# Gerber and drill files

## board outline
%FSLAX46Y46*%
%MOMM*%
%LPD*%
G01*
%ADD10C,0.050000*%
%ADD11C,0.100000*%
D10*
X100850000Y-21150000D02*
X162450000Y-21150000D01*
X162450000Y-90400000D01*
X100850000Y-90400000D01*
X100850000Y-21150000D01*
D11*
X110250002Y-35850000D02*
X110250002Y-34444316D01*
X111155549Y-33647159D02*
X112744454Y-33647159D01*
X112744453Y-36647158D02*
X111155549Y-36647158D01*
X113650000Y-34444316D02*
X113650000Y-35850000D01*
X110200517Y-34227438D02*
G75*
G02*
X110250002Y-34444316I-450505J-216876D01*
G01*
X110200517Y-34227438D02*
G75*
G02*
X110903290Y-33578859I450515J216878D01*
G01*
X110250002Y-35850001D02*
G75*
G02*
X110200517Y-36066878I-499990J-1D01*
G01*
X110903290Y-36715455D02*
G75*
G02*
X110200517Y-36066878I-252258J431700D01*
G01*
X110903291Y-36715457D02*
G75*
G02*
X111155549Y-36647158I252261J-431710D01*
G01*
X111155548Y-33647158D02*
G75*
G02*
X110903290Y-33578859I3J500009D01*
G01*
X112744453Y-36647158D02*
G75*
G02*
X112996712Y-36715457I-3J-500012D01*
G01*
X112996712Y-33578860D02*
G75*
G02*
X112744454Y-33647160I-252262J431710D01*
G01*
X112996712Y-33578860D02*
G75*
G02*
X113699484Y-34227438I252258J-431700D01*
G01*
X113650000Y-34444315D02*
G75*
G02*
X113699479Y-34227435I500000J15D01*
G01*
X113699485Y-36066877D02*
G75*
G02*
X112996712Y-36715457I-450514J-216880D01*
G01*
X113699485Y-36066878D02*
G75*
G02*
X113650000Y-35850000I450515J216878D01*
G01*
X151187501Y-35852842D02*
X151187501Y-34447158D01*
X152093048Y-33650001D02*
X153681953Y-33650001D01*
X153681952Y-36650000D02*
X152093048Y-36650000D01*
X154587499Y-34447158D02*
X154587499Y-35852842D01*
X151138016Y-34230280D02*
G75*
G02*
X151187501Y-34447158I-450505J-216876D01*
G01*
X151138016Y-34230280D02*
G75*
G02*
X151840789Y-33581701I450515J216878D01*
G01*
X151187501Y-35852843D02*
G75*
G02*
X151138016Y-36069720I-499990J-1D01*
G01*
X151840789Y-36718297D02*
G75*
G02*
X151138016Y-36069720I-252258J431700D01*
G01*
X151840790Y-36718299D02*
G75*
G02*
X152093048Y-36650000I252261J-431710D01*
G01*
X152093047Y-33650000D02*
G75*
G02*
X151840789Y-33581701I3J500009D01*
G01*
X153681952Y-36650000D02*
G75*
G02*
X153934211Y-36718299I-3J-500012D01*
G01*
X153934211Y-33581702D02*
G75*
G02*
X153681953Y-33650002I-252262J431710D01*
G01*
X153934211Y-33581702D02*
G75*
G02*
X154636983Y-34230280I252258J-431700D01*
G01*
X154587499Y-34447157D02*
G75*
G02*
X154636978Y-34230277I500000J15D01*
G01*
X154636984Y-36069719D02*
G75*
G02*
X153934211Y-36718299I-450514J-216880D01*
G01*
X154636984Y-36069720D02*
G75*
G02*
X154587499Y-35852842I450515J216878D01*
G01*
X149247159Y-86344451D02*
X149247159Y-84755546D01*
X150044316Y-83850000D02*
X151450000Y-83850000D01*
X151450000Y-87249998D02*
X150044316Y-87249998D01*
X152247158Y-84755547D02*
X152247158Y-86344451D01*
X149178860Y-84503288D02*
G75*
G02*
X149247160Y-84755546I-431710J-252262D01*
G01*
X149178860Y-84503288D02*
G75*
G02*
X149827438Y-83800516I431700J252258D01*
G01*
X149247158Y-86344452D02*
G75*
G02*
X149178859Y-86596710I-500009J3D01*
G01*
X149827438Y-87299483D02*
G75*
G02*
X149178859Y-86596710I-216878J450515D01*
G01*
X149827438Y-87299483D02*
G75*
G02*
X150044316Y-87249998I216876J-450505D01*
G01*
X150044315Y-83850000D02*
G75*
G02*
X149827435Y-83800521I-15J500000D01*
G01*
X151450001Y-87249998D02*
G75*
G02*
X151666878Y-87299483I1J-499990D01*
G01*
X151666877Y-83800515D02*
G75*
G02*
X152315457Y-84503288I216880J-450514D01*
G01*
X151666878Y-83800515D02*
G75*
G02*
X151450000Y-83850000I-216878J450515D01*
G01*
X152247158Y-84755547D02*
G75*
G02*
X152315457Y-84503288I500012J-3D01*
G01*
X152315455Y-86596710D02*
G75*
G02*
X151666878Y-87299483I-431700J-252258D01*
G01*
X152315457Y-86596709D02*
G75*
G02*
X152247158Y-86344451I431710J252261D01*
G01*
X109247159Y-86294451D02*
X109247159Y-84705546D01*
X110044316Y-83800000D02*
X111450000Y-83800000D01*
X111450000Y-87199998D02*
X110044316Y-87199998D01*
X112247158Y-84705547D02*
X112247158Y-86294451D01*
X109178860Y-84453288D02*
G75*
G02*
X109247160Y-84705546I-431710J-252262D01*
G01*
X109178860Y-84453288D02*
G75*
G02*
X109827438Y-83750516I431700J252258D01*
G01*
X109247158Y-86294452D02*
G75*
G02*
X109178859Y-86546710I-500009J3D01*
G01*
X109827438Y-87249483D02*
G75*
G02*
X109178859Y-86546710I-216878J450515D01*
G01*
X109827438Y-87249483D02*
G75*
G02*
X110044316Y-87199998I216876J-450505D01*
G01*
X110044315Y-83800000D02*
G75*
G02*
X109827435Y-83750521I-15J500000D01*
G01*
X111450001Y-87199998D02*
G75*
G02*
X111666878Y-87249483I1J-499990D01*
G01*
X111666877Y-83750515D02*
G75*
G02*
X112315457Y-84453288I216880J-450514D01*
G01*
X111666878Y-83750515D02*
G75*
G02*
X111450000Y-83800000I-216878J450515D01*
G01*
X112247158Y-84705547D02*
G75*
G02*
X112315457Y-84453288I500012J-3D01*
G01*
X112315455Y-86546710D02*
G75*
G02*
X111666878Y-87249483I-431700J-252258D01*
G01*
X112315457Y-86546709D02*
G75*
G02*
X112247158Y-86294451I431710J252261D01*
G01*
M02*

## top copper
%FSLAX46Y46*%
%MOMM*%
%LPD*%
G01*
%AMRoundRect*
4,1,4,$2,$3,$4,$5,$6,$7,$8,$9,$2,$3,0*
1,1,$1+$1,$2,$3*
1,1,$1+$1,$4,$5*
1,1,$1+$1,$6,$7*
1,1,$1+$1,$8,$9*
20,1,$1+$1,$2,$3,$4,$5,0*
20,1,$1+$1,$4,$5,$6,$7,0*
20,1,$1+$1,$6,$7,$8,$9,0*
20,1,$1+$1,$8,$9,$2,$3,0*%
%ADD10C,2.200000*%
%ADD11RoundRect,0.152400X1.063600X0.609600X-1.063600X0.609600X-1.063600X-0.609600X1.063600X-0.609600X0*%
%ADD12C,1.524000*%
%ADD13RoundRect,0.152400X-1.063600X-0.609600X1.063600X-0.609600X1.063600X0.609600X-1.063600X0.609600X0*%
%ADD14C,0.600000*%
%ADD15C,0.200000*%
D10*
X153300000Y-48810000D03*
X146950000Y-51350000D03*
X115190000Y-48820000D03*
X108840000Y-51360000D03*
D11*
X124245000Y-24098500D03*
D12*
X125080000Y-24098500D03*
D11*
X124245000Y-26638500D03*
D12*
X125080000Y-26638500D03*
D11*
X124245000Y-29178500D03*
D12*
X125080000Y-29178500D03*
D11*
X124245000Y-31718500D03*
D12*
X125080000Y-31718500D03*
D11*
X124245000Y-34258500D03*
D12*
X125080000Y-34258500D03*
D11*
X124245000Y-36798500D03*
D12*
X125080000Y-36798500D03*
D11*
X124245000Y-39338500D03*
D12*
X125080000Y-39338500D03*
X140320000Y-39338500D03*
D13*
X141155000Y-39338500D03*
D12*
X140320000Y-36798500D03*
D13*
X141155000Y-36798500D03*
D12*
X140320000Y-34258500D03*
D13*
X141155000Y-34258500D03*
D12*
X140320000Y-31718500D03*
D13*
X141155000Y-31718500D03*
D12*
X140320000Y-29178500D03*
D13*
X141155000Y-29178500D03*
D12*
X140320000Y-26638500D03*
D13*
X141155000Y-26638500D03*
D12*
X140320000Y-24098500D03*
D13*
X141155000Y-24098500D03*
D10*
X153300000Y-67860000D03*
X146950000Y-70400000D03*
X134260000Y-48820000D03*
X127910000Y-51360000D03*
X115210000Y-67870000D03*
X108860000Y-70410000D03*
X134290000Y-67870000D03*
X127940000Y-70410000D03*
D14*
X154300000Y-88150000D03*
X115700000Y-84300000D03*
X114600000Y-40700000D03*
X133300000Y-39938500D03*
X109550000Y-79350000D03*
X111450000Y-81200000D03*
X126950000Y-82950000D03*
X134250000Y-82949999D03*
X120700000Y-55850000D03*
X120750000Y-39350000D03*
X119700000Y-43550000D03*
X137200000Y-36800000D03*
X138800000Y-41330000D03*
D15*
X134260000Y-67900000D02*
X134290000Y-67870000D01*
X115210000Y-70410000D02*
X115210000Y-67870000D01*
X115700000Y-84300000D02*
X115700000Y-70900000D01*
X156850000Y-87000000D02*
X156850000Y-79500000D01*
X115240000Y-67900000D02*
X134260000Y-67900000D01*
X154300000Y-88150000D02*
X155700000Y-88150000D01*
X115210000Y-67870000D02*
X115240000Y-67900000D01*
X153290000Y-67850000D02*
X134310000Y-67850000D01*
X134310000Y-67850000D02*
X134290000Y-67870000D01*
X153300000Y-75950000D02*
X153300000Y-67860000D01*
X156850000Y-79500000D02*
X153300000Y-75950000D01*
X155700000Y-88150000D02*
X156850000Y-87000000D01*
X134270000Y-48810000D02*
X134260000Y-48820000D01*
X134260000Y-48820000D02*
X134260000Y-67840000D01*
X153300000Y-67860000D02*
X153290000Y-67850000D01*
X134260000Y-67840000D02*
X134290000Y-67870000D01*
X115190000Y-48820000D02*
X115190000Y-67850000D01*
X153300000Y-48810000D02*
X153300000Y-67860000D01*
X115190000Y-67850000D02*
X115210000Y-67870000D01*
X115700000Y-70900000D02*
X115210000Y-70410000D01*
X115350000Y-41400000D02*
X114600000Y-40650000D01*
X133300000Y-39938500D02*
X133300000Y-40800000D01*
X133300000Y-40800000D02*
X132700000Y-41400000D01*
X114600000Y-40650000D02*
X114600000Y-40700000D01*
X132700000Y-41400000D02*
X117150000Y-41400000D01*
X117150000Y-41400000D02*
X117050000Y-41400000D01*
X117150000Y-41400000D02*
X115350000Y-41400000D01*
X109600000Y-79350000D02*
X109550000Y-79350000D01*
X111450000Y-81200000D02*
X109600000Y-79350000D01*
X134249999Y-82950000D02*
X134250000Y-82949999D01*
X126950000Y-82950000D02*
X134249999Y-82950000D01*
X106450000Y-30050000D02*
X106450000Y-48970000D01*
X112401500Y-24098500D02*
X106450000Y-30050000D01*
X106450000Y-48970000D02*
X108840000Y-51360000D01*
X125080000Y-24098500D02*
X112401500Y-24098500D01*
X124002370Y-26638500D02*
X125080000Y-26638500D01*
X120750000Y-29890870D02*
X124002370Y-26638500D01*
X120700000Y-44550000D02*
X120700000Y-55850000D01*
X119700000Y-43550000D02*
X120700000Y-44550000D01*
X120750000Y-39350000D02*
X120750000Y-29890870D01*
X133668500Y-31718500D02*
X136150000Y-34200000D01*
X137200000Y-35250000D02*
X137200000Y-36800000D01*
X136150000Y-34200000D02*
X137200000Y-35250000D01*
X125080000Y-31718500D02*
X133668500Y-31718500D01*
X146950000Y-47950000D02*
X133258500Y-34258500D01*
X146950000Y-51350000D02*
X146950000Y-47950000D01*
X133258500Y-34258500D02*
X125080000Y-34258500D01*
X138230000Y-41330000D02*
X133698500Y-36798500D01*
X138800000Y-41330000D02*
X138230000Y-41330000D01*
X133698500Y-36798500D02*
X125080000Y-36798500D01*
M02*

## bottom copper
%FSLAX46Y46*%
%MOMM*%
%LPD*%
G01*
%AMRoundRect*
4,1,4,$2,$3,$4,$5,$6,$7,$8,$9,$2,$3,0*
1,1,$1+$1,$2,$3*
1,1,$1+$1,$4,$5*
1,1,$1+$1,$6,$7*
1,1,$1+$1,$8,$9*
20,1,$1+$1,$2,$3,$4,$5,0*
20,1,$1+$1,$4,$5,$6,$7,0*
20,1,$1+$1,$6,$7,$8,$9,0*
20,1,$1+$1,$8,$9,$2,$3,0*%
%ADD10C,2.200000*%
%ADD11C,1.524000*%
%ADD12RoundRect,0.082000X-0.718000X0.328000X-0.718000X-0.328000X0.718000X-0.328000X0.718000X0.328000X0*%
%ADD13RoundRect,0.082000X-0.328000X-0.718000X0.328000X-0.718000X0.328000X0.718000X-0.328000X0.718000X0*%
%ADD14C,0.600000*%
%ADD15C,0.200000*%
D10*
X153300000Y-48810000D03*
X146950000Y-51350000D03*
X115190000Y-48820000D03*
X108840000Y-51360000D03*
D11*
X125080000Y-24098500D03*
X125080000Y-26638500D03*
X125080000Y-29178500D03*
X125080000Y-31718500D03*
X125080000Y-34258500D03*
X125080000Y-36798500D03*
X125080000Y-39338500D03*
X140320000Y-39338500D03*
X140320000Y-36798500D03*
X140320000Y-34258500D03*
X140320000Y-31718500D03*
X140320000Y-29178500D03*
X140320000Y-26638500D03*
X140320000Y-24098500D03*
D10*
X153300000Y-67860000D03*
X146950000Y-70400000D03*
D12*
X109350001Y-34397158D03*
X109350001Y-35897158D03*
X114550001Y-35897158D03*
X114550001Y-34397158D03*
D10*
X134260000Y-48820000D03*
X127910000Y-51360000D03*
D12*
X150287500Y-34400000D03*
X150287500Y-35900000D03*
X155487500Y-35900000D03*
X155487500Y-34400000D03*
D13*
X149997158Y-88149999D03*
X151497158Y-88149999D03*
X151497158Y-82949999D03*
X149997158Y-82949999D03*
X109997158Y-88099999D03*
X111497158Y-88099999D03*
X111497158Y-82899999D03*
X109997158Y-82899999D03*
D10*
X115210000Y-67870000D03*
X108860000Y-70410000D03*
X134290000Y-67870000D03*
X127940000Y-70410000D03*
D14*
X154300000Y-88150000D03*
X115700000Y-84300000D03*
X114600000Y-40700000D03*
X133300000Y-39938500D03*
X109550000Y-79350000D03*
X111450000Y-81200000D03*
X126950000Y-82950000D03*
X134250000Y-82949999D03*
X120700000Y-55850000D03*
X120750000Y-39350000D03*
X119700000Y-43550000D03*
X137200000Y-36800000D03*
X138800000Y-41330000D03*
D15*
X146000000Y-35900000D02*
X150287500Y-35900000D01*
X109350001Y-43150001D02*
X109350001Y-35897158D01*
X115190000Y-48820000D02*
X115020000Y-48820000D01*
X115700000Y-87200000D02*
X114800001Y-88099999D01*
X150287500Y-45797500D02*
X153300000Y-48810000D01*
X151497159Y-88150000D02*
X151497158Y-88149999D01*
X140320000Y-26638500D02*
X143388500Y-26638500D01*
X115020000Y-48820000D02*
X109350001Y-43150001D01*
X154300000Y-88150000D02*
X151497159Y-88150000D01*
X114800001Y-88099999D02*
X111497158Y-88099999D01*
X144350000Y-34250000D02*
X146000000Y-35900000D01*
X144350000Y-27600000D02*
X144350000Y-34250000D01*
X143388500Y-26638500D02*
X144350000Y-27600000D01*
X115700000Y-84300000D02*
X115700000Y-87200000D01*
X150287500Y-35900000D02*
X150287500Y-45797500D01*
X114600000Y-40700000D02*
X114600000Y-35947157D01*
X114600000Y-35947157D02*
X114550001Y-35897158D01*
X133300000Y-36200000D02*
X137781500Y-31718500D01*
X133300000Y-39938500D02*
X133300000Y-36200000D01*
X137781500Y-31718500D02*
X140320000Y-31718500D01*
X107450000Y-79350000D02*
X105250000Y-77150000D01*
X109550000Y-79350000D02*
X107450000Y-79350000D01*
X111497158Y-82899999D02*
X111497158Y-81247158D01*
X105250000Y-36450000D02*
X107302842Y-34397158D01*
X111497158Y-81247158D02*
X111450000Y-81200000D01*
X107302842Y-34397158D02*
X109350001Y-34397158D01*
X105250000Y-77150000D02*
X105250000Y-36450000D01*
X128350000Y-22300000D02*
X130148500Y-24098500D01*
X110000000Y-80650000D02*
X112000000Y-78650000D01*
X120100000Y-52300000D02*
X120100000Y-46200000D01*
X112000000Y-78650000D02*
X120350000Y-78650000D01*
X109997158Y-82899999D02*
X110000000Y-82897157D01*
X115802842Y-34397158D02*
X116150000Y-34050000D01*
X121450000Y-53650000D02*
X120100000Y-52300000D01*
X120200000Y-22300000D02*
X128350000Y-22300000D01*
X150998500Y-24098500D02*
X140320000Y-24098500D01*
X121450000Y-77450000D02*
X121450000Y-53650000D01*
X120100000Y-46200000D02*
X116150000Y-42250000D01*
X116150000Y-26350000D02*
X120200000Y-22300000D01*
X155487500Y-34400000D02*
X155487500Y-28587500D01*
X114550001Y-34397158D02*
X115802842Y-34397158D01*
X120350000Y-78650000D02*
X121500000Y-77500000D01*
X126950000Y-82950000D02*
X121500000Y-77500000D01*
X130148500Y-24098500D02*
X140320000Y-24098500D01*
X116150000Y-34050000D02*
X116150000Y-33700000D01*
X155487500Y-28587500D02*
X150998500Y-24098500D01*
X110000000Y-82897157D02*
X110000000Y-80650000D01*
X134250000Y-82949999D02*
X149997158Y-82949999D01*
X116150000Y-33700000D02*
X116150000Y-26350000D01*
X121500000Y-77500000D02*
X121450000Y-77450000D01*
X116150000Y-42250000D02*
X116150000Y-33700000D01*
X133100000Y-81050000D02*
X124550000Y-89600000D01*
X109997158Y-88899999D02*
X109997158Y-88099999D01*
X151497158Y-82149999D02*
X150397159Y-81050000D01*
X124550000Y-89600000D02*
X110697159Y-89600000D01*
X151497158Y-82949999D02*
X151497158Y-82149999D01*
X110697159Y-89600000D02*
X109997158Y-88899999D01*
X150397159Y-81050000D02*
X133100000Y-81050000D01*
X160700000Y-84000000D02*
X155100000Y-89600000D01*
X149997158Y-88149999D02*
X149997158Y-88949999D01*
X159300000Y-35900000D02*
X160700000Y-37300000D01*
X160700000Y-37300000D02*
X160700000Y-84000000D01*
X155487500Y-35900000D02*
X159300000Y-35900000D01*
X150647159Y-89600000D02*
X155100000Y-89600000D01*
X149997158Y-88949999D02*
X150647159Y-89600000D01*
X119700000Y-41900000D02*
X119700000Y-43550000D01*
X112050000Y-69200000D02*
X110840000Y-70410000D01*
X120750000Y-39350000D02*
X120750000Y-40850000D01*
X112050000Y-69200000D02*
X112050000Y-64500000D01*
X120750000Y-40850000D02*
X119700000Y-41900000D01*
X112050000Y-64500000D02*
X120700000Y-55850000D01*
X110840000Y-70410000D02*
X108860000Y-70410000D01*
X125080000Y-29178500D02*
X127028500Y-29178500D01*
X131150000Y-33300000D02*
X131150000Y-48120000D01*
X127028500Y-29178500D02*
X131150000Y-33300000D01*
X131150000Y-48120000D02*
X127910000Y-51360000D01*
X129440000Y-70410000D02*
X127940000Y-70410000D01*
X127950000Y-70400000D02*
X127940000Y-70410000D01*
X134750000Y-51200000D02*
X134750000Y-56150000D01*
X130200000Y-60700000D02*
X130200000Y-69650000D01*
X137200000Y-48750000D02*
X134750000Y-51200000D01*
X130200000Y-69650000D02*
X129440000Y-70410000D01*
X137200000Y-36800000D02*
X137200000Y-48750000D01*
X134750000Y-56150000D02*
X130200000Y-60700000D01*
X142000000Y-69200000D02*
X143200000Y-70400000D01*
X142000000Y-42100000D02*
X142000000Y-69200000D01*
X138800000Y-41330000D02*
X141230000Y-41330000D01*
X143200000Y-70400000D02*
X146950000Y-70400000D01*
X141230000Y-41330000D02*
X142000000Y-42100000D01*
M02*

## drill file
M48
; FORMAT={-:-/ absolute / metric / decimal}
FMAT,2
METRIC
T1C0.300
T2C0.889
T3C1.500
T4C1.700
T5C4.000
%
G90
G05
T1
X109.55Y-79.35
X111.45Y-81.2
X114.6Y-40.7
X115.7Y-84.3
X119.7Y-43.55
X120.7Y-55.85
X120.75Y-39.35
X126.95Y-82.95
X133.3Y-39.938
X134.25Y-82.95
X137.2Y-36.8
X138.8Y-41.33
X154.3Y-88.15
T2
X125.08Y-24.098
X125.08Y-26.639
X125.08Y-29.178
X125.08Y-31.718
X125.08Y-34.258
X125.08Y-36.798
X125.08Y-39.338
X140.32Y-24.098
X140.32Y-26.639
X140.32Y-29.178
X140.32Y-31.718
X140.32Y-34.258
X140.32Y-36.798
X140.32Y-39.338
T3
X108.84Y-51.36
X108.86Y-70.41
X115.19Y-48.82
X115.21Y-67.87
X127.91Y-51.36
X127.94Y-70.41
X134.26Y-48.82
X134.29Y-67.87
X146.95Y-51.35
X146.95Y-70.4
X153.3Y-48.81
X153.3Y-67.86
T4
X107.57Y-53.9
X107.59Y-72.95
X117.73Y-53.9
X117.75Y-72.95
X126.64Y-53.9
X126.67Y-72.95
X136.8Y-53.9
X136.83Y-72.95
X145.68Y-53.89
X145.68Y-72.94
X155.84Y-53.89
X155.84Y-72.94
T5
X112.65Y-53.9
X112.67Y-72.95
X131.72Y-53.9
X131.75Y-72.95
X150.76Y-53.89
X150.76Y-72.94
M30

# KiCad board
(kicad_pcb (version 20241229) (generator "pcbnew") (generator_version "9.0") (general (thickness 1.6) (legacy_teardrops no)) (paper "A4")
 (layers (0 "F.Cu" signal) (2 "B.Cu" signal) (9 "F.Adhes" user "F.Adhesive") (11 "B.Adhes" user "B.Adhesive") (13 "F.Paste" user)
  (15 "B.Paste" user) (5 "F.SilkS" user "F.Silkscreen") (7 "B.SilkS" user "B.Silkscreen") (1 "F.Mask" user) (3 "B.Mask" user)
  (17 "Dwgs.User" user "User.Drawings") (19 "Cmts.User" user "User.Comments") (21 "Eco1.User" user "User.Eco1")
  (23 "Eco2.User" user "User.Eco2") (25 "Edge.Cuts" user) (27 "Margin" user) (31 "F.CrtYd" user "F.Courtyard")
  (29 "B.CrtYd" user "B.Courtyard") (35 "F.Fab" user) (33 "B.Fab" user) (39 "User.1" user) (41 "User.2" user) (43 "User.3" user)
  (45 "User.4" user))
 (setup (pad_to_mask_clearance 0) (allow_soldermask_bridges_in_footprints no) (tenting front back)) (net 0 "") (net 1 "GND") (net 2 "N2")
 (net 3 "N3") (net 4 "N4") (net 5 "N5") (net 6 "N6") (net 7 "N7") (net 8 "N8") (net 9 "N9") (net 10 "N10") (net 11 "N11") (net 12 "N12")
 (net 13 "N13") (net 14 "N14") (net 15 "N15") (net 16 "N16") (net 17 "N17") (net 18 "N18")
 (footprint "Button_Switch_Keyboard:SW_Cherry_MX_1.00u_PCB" (layer "F.Cu") (at 153.3 48.81)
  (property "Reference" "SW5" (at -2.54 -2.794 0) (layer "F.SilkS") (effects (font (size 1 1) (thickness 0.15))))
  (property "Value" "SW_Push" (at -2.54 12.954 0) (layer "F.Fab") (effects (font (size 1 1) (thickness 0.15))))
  (pad "" np_thru_hole circle (at -7.62 5.08) (size 1.7 1.7) (drill 1.7) (layers "*.Cu" "*.Mask"))
  (pad "" np_thru_hole circle (at -2.54 5.08) (size 4 4) (drill 4) (layers "*.Cu" "*.Mask"))
  (pad "" np_thru_hole circle (at 2.54 5.08) (size 1.7 1.7) (drill 1.7) (layers "*.Cu" "*.Mask"))
  (pad "1" thru_hole circle (at 0 0) (size 2.2 2.2) (drill 1.5) (layers "*.Cu" "*.Mask") (remove_unused_layers no) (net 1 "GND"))
  (pad "2" thru_hole circle (at -6.35 2.54) (size 2.2 2.2) (drill 1.5) (layers "*.Cu" "*.Mask") (remove_unused_layers no) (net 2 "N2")))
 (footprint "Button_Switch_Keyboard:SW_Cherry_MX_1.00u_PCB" (layer "F.Cu") (at 115.19 48.82)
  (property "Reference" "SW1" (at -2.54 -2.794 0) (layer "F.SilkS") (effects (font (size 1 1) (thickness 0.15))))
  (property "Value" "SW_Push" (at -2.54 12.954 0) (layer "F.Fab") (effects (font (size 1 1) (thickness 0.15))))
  (pad "" np_thru_hole circle (at -7.62 5.08) (size 1.7 1.7) (drill 1.7) (layers "*.Cu" "*.Mask"))
  (pad "" np_thru_hole circle (at -2.54 5.08) (size 4 4) (drill 4) (layers "*.Cu" "*.Mask"))
  (pad "" np_thru_hole circle (at 2.54 5.08) (size 1.7 1.7) (drill 1.7) (layers "*.Cu" "*.Mask"))
  (pad "1" thru_hole circle (at 0 0) (size 2.2 2.2) (drill 1.5) (layers "*.Cu" "*.Mask") (remove_unused_layers no) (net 1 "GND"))
  (pad "2" thru_hole circle (at -6.35 2.54) (size 2.2 2.2) (drill 1.5) (layers "*.Cu" "*.Mask") (remove_unused_layers no) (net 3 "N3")))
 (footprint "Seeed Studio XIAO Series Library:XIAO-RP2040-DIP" (layer "F.Cu") (at 132.7 31.7185)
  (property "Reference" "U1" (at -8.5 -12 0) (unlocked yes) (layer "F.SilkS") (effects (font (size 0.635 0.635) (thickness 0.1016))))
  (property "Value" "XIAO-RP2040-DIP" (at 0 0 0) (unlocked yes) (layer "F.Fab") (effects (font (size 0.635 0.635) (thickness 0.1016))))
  (pad "1" smd roundrect (at -8.455 -7.62 180) (size 2.432 1.524) (layers "F.Cu" "F.Mask") (roundrect_rratio 0.1) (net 3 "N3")
   (thermal_bridge_angle 45))
  (pad "1" thru_hole circle (at -7.62 -7.62 180) (size 1.524 1.524) (drill 0.889) (layers "*.Cu" "*.Mask") (remove_unused_layers no)
   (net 3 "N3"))
  (pad "2" smd roundrect (at -8.455 -5.08 180) (size 2.432 1.524) (layers "F.Cu" "F.Mask") (roundrect_rratio 0.1) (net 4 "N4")
   (thermal_bridge_angle 45))
  (pad "2" thru_hole circle (at -7.62 -5.08 180) (size 1.524 1.524) (drill 0.889) (layers "*.Cu" "*.Mask") (remove_unused_layers no)
   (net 4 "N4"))
  (pad "3" smd roundrect (at -8.455 -2.54 180) (size 2.432 1.524) (layers "F.Cu" "F.Mask") (roundrect_rratio 0.1) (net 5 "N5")
   (thermal_bridge_angle 45))
  (pad "3" thru_hole circle (at -7.62 -2.54 180) (size 1.524 1.524) (drill 0.889) (layers "*.Cu" "*.Mask") (remove_unused_layers no)
   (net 5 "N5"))
  (pad "4" smd roundrect (at -8.455 0 180) (size 2.432 1.524) (layers "F.Cu" "F.Mask") (roundrect_rratio 0.1) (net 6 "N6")
   (thermal_bridge_angle 45))
  (pad "4" thru_hole circle (at -7.62 0 180) (size 1.524 1.524) (drill 0.889) (layers "*.Cu" "*.Mask") (remove_unused_layers no)
   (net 6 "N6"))
  (pad "5" smd roundrect (at -8.455 2.54 180) (size 2.432 1.524) (layers "F.Cu" "F.Mask") (roundrect_rratio 0.1) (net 2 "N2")
   (thermal_bridge_angle 45))
  (pad "5" thru_hole circle (at -7.62 2.54 180) (size 1.524 1.524) (drill 0.889) (layers "*.Cu" "*.Mask") (remove_unused_layers no)
   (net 2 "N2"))
  (pad "6" smd roundrect (at -8.455 5.08 180) (size 2.432 1.524) (layers "F.Cu" "F.Mask") (roundrect_rratio 0.1) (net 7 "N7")
   (thermal_bridge_angle 45))
  (pad "6" thru_hole circle (at -7.62 5.08 180) (size 1.524 1.524) (drill 0.889) (layers "*.Cu" "*.Mask") (remove_unused_layers no)
   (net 7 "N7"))
  (pad "7" smd roundrect (at -8.455 7.62 180) (size 2.432 1.524) (layers "F.Cu" "F.Mask") (roundrect_rratio 0.1) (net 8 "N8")
   (thermal_bridge_angle 45))
  (pad "7" thru_hole circle (at -7.62 7.62 180) (size 1.524 1.524) (drill 0.889) (layers "*.Cu" "*.Mask") (remove_unused_layers no)
   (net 8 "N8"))
  (pad "8" thru_hole circle (at 7.62 7.62) (size 1.524 1.524) (drill 0.889) (layers "*.Cu" "*.Mask") (remove_unused_layers no) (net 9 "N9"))
  (pad "8" smd roundrect (at 8.455 7.62) (size 2.432 1.524) (layers "F.Cu" "F.Mask") (roundrect_rratio 0.1) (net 9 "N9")
   (thermal_bridge_angle 45))
  (pad "9" thru_hole circle (at 7.62 5.08) (size 1.524 1.524) (drill 0.889) (layers "*.Cu" "*.Mask") (remove_unused_layers no)
   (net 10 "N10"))
  (pad "9" smd roundrect (at 8.455 5.08) (size 2.432 1.524) (layers "F.Cu" "F.Mask") (roundrect_rratio 0.1) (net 10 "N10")
   (thermal_bridge_angle 45))
  (pad "10" thru_hole circle (at 7.62 2.54) (size 1.524 1.524) (drill 0.889) (layers "*.Cu" "*.Mask") (remove_unused_layers no)
   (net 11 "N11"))
  (pad "10" smd roundrect (at 8.455 2.54) (size 2.432 1.524) (layers "F.Cu" "F.Mask") (roundrect_rratio 0.1) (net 11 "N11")
   (thermal_bridge_angle 45))
  (pad "11" thru_hole circle (at 7.62 0) (size 1.524 1.524) (drill 0.889) (layers "*.Cu" "*.Mask") (remove_unused_layers no) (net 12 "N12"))
  (pad "11" smd roundrect (at 8.455 0) (size 2.432 1.524) (layers "F.Cu" "F.Mask") (roundrect_rratio 0.1) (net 12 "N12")
   (thermal_bridge_angle 45))
  (pad "12" thru_hole circle (at 7.62 -2.54) (size 1.524 1.524) (drill 0.889) (layers "*.Cu" "*.Mask") (remove_unused_layers no)
   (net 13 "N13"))
  (pad "12" smd roundrect (at 8.455 -2.54) (size 2.432 1.524) (layers "F.Cu" "F.Mask") (roundrect_rratio 0.1) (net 13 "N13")
   (thermal_bridge_angle 45))
  (pad "13" thru_hole circle (at 7.62 -5.08) (size 1.524 1.524) (drill 0.889) (layers "*.Cu" "*.Mask") (remove_unused_layers no)
   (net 1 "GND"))
  (pad "13" smd roundrect (at 8.455 -5.08) (size 2.432 1.524) (layers "F.Cu" "F.Mask") (roundrect_rratio 0.1) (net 1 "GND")
   (thermal_bridge_angle 45))
  (pad "14" thru_hole circle (at 7.62 -7.62) (size 1.524 1.524) (drill 0.889) (layers "*.Cu" "*.Mask") (remove_unused_layers no)
   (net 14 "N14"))
  (pad "14" smd roundrect (at 8.455 -7.62) (size 2.432 1.524) (layers "F.Cu" "F.Mask") (roundrect_rratio 0.1) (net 14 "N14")
   (thermal_bridge_angle 45)))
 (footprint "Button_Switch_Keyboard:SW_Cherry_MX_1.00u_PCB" (layer "F.Cu") (at 153.3 67.86)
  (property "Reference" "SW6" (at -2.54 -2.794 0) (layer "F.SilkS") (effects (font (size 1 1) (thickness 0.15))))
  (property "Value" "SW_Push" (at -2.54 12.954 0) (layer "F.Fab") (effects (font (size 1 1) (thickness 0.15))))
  (pad "" np_thru_hole circle (at -7.62 5.08) (size 1.7 1.7) (drill 1.7) (layers "*.Cu" "*.Mask"))
  (pad "" np_thru_hole circle (at -2.54 5.08) (size 4 4) (drill 4) (layers "*.Cu" "*.Mask"))
  (pad "" np_thru_hole circle (at 2.54 5.08) (size 1.7 1.7) (drill 1.7) (layers "*.Cu" "*.Mask"))
  (pad "1" thru_hole circle (at 0 0) (size 2.2 2.2) (drill 1.5) (layers "*.Cu" "*.Mask") (remove_unused_layers no) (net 1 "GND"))
  (pad "2" thru_hole circle (at -6.35 2.54) (size 2.2 2.2) (drill 1.5) (layers "*.Cu" "*.Mask") (remove_unused_layers no) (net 7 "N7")))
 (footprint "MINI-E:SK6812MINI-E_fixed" (layer "F.Cu") (at 111.95 35.25)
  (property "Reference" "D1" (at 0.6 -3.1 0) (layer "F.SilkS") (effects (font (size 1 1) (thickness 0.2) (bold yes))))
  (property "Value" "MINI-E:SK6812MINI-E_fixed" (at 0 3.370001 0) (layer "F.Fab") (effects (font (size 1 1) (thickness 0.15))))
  (fp_line (start -1.699998 0.6) (end -1.699998 -0.805684) (stroke (width 0.1) (type solid)) (layer "Edge.Cuts"))
  (fp_line (start -0.794451 -1.602841) (end 0.794454 -1.602841) (stroke (width 0.1) (type solid)) (layer "Edge.Cuts"))
  (fp_line (start 0.794453 1.397158) (end -0.794451 1.397158) (stroke (width 0.1) (type solid)) (layer "Edge.Cuts"))
  (fp_line (start 1.7 -0.805684) (end 1.7 0.6) (stroke (width 0.1) (type solid)) (layer "Edge.Cuts"))
  (fp_arc (start -1.749483 -1.022562) (mid -1.712526 -0.91691) (end -1.699998 -0.805684) (stroke (width 0.1) (type solid))
   (layer "Edge.Cuts"))
  (fp_arc (start -1.749483 -1.022562) (mid -1.63807 -1.606877) (end -1.04671 -1.671141) (stroke (width 0.1) (type solid))
   (layer "Edge.Cuts"))
  (fp_arc (start -1.699998 0.600001) (mid -1.712526 0.711226) (end -1.749483 0.816878) (stroke (width 0.1) (type solid)) (layer "Edge.Cuts"))
  (fp_arc (start -1.04671 1.465455) (mid -1.638069 1.401192) (end -1.749483 0.816878) (stroke (width 0.1) (type solid)) (layer "Edge.Cuts"))
  (fp_arc (start -1.046709 1.465457) (mid -0.925121 1.414535) (end -0.794451 1.397158) (stroke (width 0.1) (type solid)) (layer "Edge.Cuts"))
  (fp_arc (start -0.794452 -1.602842) (mid -0.925122 -1.620219) (end -1.04671 -1.671141) (stroke (width 0.1) (type solid))
   (layer "Edge.Cuts"))
  (fp_arc (start 0.794453 1.397158) (mid 0.925124 1.414535) (end 1.046712 1.465457) (stroke (width 0.1) (type solid)) (layer "Edge.Cuts"))
  (fp_arc (start 1.046712 -1.67114) (mid 0.925124 -1.620218) (end 0.794454 -1.602841) (stroke (width 0.1) (type solid)) (layer "Edge.Cuts"))
  (fp_arc (start 1.046712 -1.67114) (mid 1.638072 -1.606876) (end 1.749485 -1.022562) (stroke (width 0.1) (type solid)) (layer "Edge.Cuts"))
  (fp_arc (start 1.7 -0.805685) (mid 1.712528 -0.91691) (end 1.749485 -1.022562) (stroke (width 0.1) (type solid)) (layer "Edge.Cuts"))
  (fp_arc (start 1.749485 0.816877) (mid 1.638073 1.401193) (end 1.046712 1.465457) (stroke (width 0.1) (type solid)) (layer "Edge.Cuts"))
  (fp_arc (start 1.749485 0.816878) (mid 1.712528 0.711226) (end 1.7 0.6) (stroke (width 0.1) (type solid)) (layer "Edge.Cuts"))
  (pad "1" smd roundrect (at -2.599999 -0.852842 270) (size 0.82 1.6) (layers "B.Cu" "B.Mask" "B.Paste") (roundrect_rratio 0.1)
   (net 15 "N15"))
  (pad "2" smd roundrect (at -2.599999 0.647158 270) (size 0.82 1.6) (layers "B.Cu" "B.Mask" "B.Paste") (roundrect_rratio 0.1) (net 1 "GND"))
  (pad "3" smd roundrect (at 2.600001 0.647158 270) (size 0.82 1.6) (layers "B.Cu" "B.Mask" "B.Paste") (roundrect_rratio 0.1) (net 12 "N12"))
  (pad "4" smd roundrect (at 2.600001 -0.852842 270) (size 0.82 1.6) (layers "B.Cu" "B.Mask" "B.Paste") (roundrect_rratio 0.1)
   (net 14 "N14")))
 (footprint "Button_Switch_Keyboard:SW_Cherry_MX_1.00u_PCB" (layer "F.Cu") (at 134.26 48.82)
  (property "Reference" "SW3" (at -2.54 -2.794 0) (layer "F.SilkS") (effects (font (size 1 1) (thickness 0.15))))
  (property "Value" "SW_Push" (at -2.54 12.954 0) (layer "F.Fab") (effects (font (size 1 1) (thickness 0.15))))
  (pad "" np_thru_hole circle (at -7.62 5.08) (size 1.7 1.7) (drill 1.7) (layers "*.Cu" "*.Mask"))
  (pad "" np_thru_hole circle (at -2.54 5.08) (size 4 4) (drill 4) (layers "*.Cu" "*.Mask"))
  (pad "" np_thru_hole circle (at 2.54 5.08) (size 1.7 1.7) (drill 1.7) (layers "*.Cu" "*.Mask"))
  (pad "1" thru_hole circle (at 0 0) (size 2.2 2.2) (drill 1.5) (layers "*.Cu" "*.Mask") (remove_unused_layers no) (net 1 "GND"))
  (pad "2" thru_hole circle (at -6.35 2.54) (size 2.2 2.2) (drill 1.5) (layers "*.Cu" "*.Mask") (remove_unused_layers no) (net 5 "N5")))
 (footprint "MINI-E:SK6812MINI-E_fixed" (layer "F.Cu") (at 152.887499 35.252842)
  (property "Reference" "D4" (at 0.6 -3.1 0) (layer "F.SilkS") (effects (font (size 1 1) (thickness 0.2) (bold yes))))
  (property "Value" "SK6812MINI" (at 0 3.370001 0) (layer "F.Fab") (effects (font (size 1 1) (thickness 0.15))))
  (fp_line (start -1.699998 0.6) (end -1.699998 -0.805684) (stroke (width 0.1) (type solid)) (layer "Edge.Cuts"))
  (fp_line (start -0.794451 -1.602841) (end 0.794454 -1.602841) (stroke (width 0.1) (type solid)) (layer "Edge.Cuts"))
  (fp_line (start 0.794453 1.397158) (end -0.794451 1.397158) (stroke (width 0.1) (type solid)) (layer "Edge.Cuts"))
  (fp_line (start 1.7 -0.805684) (end 1.7 0.6) (stroke (width 0.1) (type solid)) (layer "Edge.Cuts"))
  (fp_arc (start -1.749483 -1.022562) (mid -1.712526 -0.91691) (end -1.699998 -0.805684) (stroke (width 0.1) (type solid))
   (layer "Edge.Cuts"))
  (fp_arc (start -1.749483 -1.022562) (mid -1.63807 -1.606877) (end -1.04671 -1.671141) (stroke (width 0.1) (type solid))
   (layer "Edge.Cuts"))
  (fp_arc (start -1.699998 0.600001) (mid -1.712526 0.711226) (end -1.749483 0.816878) (stroke (width 0.1) (type solid)) (layer "Edge.Cuts"))
  (fp_arc (start -1.04671 1.465455) (mid -1.638069 1.401192) (end -1.749483 0.816878) (stroke (width 0.1) (type solid)) (layer "Edge.Cuts"))
  (fp_arc (start -1.046709 1.465457) (mid -0.925121 1.414535) (end -0.794451 1.397158) (stroke (width 0.1) (type solid)) (layer "Edge.Cuts"))
  (fp_arc (start -0.794452 -1.602842) (mid -0.925122 -1.620219) (end -1.04671 -1.671141) (stroke (width 0.1) (type solid))
   (layer "Edge.Cuts"))
  (fp_arc (start 0.794453 1.397158) (mid 0.925124 1.414535) (end 1.046712 1.465457) (stroke (width 0.1) (type solid)) (layer "Edge.Cuts"))
  (fp_arc (start 1.046712 -1.67114) (mid 0.925124 -1.620218) (end 0.794454 -1.602841) (stroke (width 0.1) (type solid)) (layer "Edge.Cuts"))
  (fp_arc (start 1.046712 -1.67114) (mid 1.638072 -1.606876) (end 1.749485 -1.022562) (stroke (width 0.1) (type solid)) (layer "Edge.Cuts"))
  (fp_arc (start 1.7 -0.805685) (mid 1.712528 -0.91691) (end 1.749485 -1.022562) (stroke (width 0.1) (type solid)) (layer "Edge.Cuts"))
  (fp_arc (start 1.749485 0.816877) (mid 1.638073 1.401193) (end 1.046712 1.465457) (stroke (width 0.1) (type solid)) (layer "Edge.Cuts"))
  (fp_arc (start 1.749485 0.816878) (mid 1.712528 0.711226) (end 1.7 0.6) (stroke (width 0.1) (type solid)) (layer "Edge.Cuts"))
  (pad "1" smd roundrect (at -2.599999 -0.852842 270) (size 0.82 1.6) (layers "B.Cu" "B.Mask" "B.Paste") (roundrect_rratio 0.1)
   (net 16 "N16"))
  (pad "2" smd roundrect (at -2.599999 0.647158 270) (size 0.82 1.6) (layers "B.Cu" "B.Mask" "B.Paste") (roundrect_rratio 0.1) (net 1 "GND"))
  (pad "3" smd roundrect (at 2.600001 0.647158 270) (size 0.82 1.6) (layers "B.Cu" "B.Mask" "B.Paste") (roundrect_rratio 0.1) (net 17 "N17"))
  (pad "4" smd roundrect (at 2.600001 -0.852842 270) (size 0.82 1.6) (layers "B.Cu" "B.Mask" "B.Paste") (roundrect_rratio 0.1)
   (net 14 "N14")))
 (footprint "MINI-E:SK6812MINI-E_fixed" (layer "F.Cu") (at 150.85 85.55 90)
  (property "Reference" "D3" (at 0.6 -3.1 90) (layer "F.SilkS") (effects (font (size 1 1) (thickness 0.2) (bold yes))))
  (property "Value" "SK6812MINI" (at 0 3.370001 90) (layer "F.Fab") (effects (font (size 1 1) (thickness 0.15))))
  (fp_line (start -0.794451 -1.602841) (end 0.794454 -1.602841) (stroke (width 0.1) (type solid)) (layer "Edge.Cuts"))
  (fp_line (start 1.7 -0.805684) (end 1.7 0.6) (stroke (width 0.1) (type solid)) (layer "Edge.Cuts"))
  (fp_line (start -1.699998 0.6) (end -1.699998 -0.805684) (stroke (width 0.1) (type solid)) (layer "Edge.Cuts"))
  (fp_line (start 0.794453 1.397158) (end -0.794451 1.397158) (stroke (width 0.1) (type solid)) (layer "Edge.Cuts"))
  (fp_arc (start 1.046712 -1.67114) (mid 0.925124 -1.620218) (end 0.794454 -1.602841) (stroke (width 0.1) (type solid)) (layer "Edge.Cuts"))
  (fp_arc (start 1.046712 -1.67114) (mid 1.638072 -1.606876) (end 1.749485 -1.022562) (stroke (width 0.1) (type solid)) (layer "Edge.Cuts"))
  (fp_arc (start -0.794452 -1.602842) (mid -0.925122 -1.620219) (end -1.04671 -1.671141) (stroke (width 0.1) (type solid))
   (layer "Edge.Cuts"))
  (fp_arc (start -1.749483 -1.022562) (mid -1.63807 -1.606877) (end -1.04671 -1.671141) (stroke (width 0.1) (type solid))
   (layer "Edge.Cuts"))
  (fp_arc (start -1.749483 -1.022562) (mid -1.712526 -0.91691) (end -1.699998 -0.805684) (stroke (width 0.1) (type solid))
   (layer "Edge.Cuts"))
  (fp_arc (start 1.7 -0.805685) (mid 1.712528 -0.91691) (end 1.749485 -1.022562) (stroke (width 0.1) (type solid)) (layer "Edge.Cuts"))
  (fp_arc (start -1.699998 0.600001) (mid -1.712526 0.711226) (end -1.749483 0.816878) (stroke (width 0.1) (type solid)) (layer "Edge.Cuts"))
  (fp_arc (start 1.749485 0.816877) (mid 1.638073 1.401193) (end 1.046712 1.465457) (stroke (width 0.1) (type solid)) (layer "Edge.Cuts"))
  (fp_arc (start 1.749485 0.816878) (mid 1.712528 0.711226) (end 1.7 0.6) (stroke (width 0.1) (type solid)) (layer "Edge.Cuts"))
  (fp_arc (start 0.794453 1.397158) (mid 0.925124 1.414535) (end 1.046712 1.465457) (stroke (width 0.1) (type solid)) (layer "Edge.Cuts"))
  (fp_arc (start -1.04671 1.465455) (mid -1.638069 1.401192) (end -1.749483 0.816878) (stroke (width 0.1) (type solid)) (layer "Edge.Cuts"))
  (fp_arc (start -1.046709 1.465457) (mid -0.925121 1.414535) (end -0.794451 1.397158) (stroke (width 0.1) (type solid)) (layer "Edge.Cuts"))
  (pad "1" smd roundrect (at -2.599999 -0.852842) (size 0.82 1.6) (layers "B.Cu" "B.Mask" "B.Paste") (roundrect_rratio 0.1) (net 17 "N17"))
  (pad "2" smd roundrect (at -2.599999 0.647158) (size 0.82 1.6) (layers "B.Cu" "B.Mask" "B.Paste") (roundrect_rratio 0.1) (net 1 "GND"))
  (pad "3" smd roundrect (at 2.600001 0.647158) (size 0.82 1.6) (layers "B.Cu" "B.Mask" "B.Paste") (roundrect_rratio 0.1) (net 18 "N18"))
  (pad "4" smd roundrect (at 2.600001 -0.852842) (size 0.82 1.6) (layers "B.Cu" "B.Mask" "B.Paste") (roundrect_rratio 0.1) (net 14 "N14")))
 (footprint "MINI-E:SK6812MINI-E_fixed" (layer "F.Cu") (at 110.85 85.5 90)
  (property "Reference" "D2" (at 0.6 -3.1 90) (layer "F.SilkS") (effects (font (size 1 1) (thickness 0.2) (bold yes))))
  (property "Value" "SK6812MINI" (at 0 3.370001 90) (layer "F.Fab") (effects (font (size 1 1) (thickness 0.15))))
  (fp_line (start -0.794451 -1.602841) (end 0.794454 -1.602841) (stroke (width 0.1) (type solid)) (layer "Edge.Cuts"))
  (fp_line (start 1.7 -0.805684) (end 1.7 0.6) (stroke (width 0.1) (type solid)) (layer "Edge.Cuts"))
  (fp_line (start -1.699998 0.6) (end -1.699998 -0.805684) (stroke (width 0.1) (type solid)) (layer "Edge.Cuts"))
  (fp_line (start 0.794453 1.397158) (end -0.794451 1.397158) (stroke (width 0.1) (type solid)) (layer "Edge.Cuts"))
  (fp_arc (start 1.046712 -1.67114) (mid 0.925124 -1.620218) (end 0.794454 -1.602841) (stroke (width 0.1) (type solid)) (layer "Edge.Cuts"))
  (fp_arc (start 1.046712 -1.67114) (mid 1.638072 -1.606876) (end 1.749485 -1.022562) (stroke (width 0.1) (type solid)) (layer "Edge.Cuts"))
  (fp_arc (start -0.794452 -1.602842) (mid -0.925122 -1.620219) (end -1.04671 -1.671141) (stroke (width 0.1) (type solid))
   (layer "Edge.Cuts"))
  (fp_arc (start -1.749483 -1.022562) (mid -1.63807 -1.606877) (end -1.04671 -1.671141) (stroke (width 0.1) (type solid))
   (layer "Edge.Cuts"))
  (fp_arc (start -1.749483 -1.022562) (mid -1.712526 -0.91691) (end -1.699998 -0.805684) (stroke (width 0.1) (type solid))
   (layer "Edge.Cuts"))
  (fp_arc (start 1.7 -0.805685) (mid 1.712528 -0.91691) (end 1.749485 -1.022562) (stroke (width 0.1) (type solid)) (layer "Edge.Cuts"))
  (fp_arc (start -1.699998 0.600001) (mid -1.712526 0.711226) (end -1.749483 0.816878) (stroke (width 0.1) (type solid)) (layer "Edge.Cuts"))
  (fp_arc (start 1.749485 0.816877) (mid 1.638073 1.401193) (end 1.046712 1.465457) (stroke (width 0.1) (type solid)) (layer "Edge.Cuts"))
  (fp_arc (start 1.749485 0.816878) (mid 1.712528 0.711226) (end 1.7 0.6) (stroke (width 0.1) (type solid)) (layer "Edge.Cuts"))
  (fp_arc (start 0.794453 1.397158) (mid 0.925124 1.414535) (end 1.046712 1.465457) (stroke (width 0.1) (type solid)) (layer "Edge.Cuts"))
  (fp_arc (start -1.04671 1.465455) (mid -1.638069 1.401192) (end -1.749483 0.816878) (stroke (width 0.1) (type solid)) (layer "Edge.Cuts"))
  (fp_arc (start -1.046709 1.465457) (mid -0.925121 1.414535) (end -0.794451 1.397158) (stroke (width 0.1) (type solid)) (layer "Edge.Cuts"))
  (pad "1" smd roundrect (at -2.599999 -0.852842) (size 0.82 1.6) (layers "B.Cu" "B.Mask" "B.Paste") (roundrect_rratio 0.1) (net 18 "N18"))
  (pad "2" smd roundrect (at -2.599999 0.647158) (size 0.82 1.6) (layers "B.Cu" "B.Mask" "B.Paste") (roundrect_rratio 0.1) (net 1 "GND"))
  (pad "3" smd roundrect (at 2.600001 0.647158) (size 0.82 1.6) (layers "B.Cu" "B.Mask" "B.Paste") (roundrect_rratio 0.1) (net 15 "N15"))
  (pad "4" smd roundrect (at 2.600001 -0.852842) (size 0.82 1.6) (layers "B.Cu" "B.Mask" "B.Paste") (roundrect_rratio 0.1) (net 14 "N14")))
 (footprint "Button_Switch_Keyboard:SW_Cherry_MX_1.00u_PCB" (layer "F.Cu") (at 115.21 67.87)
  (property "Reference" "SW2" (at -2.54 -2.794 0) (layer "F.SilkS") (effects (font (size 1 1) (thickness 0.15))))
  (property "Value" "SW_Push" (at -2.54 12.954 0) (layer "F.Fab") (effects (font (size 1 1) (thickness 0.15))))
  (pad "" np_thru_hole circle (at -7.62 5.08) (size 1.7 1.7) (drill 1.7) (layers "*.Cu" "*.Mask"))
  (pad "" np_thru_hole circle (at -2.54 5.08) (size 4 4) (drill 4) (layers "*.Cu" "*.Mask"))
  (pad "" np_thru_hole circle (at 2.54 5.08) (size 1.7 1.7) (drill 1.7) (layers "*.Cu" "*.Mask"))
  (pad "1" thru_hole circle (at 0 0) (size 2.2 2.2) (drill 1.5) (layers "*.Cu" "*.Mask") (remove_unused_layers no) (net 1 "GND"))
  (pad "2" thru_hole circle (at -6.35 2.54) (size 2.2 2.2) (drill 1.5) (layers "*.Cu" "*.Mask") (remove_unused_layers no) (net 4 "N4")))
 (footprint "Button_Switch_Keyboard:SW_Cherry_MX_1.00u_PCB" (layer "F.Cu") (at 134.29 67.87)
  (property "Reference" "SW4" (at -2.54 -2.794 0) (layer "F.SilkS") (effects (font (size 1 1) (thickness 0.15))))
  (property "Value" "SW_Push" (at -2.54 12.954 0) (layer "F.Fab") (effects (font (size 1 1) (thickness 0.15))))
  (pad "" np_thru_hole circle (at -7.62 5.08) (size 1.7 1.7) (drill 1.7) (layers "*.Cu" "*.Mask"))
  (pad "" np_thru_hole circle (at -2.54 5.08) (size 4 4) (drill 4) (layers "*.Cu" "*.Mask"))
  (pad "" np_thru_hole circle (at 2.54 5.08) (size 1.7 1.7) (drill 1.7) (layers "*.Cu" "*.Mask"))
  (pad "1" thru_hole circle (at 0 0) (size 2.2 2.2) (drill 1.5) (layers "*.Cu" "*.Mask") (remove_unused_layers no) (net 1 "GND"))
  (pad "2" thru_hole circle (at -6.35 2.54) (size 2.2 2.2) (drill 1.5) (layers "*.Cu" "*.Mask") (remove_unused_layers no) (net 6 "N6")))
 (gr_rect (start 100.85 21.15) (end 162.45 90.4) (stroke (width 0.05) (type default)) (fill no) (layer "Edge.Cuts"))
 (segment (start 134.26 67.9) (end 134.29 67.87) (width 0.2) (layer "F.Cu") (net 1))
 (segment (start 115.21 70.41) (end 115.21 67.87) (width 0.2) (layer "F.Cu") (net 1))
 (segment (start 115.7 84.3) (end 115.7 70.9) (width 0.2) (layer "F.Cu") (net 1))
 (segment (start 156.85 87) (end 156.85 79.5) (width 0.2) (layer "F.Cu") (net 1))
 (segment (start 115.24 67.9) (end 134.26 67.9) (width 0.2) (layer "F.Cu") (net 1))
 (segment (start 154.3 88.15) (end 155.7 88.15) (width 0.2) (layer "F.Cu") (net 1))
 (segment (start 115.21 67.87) (end 115.24 67.9) (width 0.2) (layer "F.Cu") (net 1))
 (segment (start 153.29 67.85) (end 134.31 67.85) (width 0.2) (layer "F.Cu") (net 1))
 (segment (start 134.31 67.85) (end 134.29 67.87) (width 0.2) (layer "F.Cu") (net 1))
 (segment (start 153.3 75.95) (end 153.3 67.86) (width 0.2) (layer "F.Cu") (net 1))
 (segment (start 156.85 79.5) (end 153.3 75.95) (width 0.2) (layer "F.Cu") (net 1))
 (segment (start 155.7 88.15) (end 156.85 87) (width 0.2) (layer "F.Cu") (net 1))
 (segment (start 134.27 48.81) (end 134.26 48.82) (width 0.2) (layer "F.Cu") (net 1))
 (segment (start 134.26 48.82) (end 134.26 67.84) (width 0.2) (layer "F.Cu") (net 1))
 (segment (start 153.3 67.86) (end 153.29 67.85) (width 0.2) (layer "F.Cu") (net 1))
 (segment (start 134.26 67.84) (end 134.29 67.87) (width 0.2) (layer "F.Cu") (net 1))
 (segment (start 115.19 48.82) (end 115.19 67.85) (width 0.2) (layer "F.Cu") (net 1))
 (segment (start 153.3 48.81) (end 153.3 67.86) (width 0.2) (layer "F.Cu") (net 1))
 (segment (start 115.19 67.85) (end 115.21 67.87) (width 0.2) (layer "F.Cu") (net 1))
 (segment (start 115.7 70.9) (end 115.21 70.41) (width 0.2) (layer "F.Cu") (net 1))
 (via (at 154.3 88.15) (size 0.6) (drill 0.3) (layers "F.Cu" "B.Cu") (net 1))
 (via (at 115.7 84.3) (size 0.6) (drill 0.3) (layers "F.Cu" "B.Cu") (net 1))
 (segment (start 146 35.9) (end 150.2875 35.9) (width 0.2) (layer "B.Cu") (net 1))
 (segment (start 109.350001 43.150001) (end 109.350001 35.897158) (width 0.2) (layer "B.Cu") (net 1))
 (segment (start 115.19 48.82) (end 115.02 48.82) (width 0.2) (layer "B.Cu") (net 1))
 (segment (start 115.7 87.2) (end 114.800001 88.099999) (width 0.2) (layer "B.Cu") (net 1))
 (segment (start 150.2875 45.7975) (end 153.3 48.81) (width 0.2) (layer "B.Cu") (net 1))
 (segment (start 151.497159 88.15) (end 151.497158 88.149999) (width 0.2) (layer "B.Cu") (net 1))
 (segment (start 140.32 26.6385) (end 143.3885 26.6385) (width 0.2) (layer "B.Cu") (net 1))
 (segment (start 115.02 48.82) (end 109.350001 43.150001) (width 0.2) (layer "B.Cu") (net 1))
 (segment (start 154.3 88.15) (end 151.497159 88.15) (width 0.2) (layer "B.Cu") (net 1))
 (segment (start 114.800001 88.099999) (end 111.497158 88.099999) (width 0.2) (layer "B.Cu") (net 1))
 (segment (start 144.35 34.25) (end 146 35.9) (width 0.2) (layer "B.Cu") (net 1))
 (segment (start 144.35 27.6) (end 144.35 34.25) (width 0.2) (layer "B.Cu") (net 1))
 (segment (start 143.3885 26.6385) (end 144.35 27.6) (width 0.2) (layer "B.Cu") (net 1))
 (segment (start 115.7 84.3) (end 115.7 87.2) (width 0.2) (layer "B.Cu") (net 1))
 (segment (start 150.2875 35.9) (end 150.2875 45.7975) (width 0.2) (layer "B.Cu") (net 1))
 (segment (start 115.35 41.4) (end 114.6 40.65) (width 0.2) (layer "F.Cu") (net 12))
 (segment (start 133.3 39.9385) (end 133.3 40.8) (width 0.2) (layer "F.Cu") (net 12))
 (segment (start 133.3 40.8) (end 132.7 41.4) (width 0.2) (layer "F.Cu") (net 12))
 (segment (start 114.6 40.65) (end 114.6 40.7) (width 0.2) (layer "F.Cu") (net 12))
 (segment (start 132.7 41.4) (end 117.15 41.4) (width 0.2) (layer "F.Cu") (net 12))
 (segment (start 117.15 41.4) (end 117.05 41.4) (width 0.2) (layer "F.Cu") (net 12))
 (segment (start 117.15 41.4) (end 115.35 41.4) (width 0.2) (layer "F.Cu") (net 12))
 (via (at 114.6 40.7) (size 0.6) (drill 0.3) (layers "F.Cu" "B.Cu") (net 12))
 (via (at 133.3 39.9385) (size 0.6) (drill 0.3) (layers "F.Cu" "B.Cu") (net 12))
 (segment (start 114.6 40.7) (end 114.6 35.947157) (width 0.2) (layer "B.Cu") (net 12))
 (segment (start 114.6 35.947157) (end 114.550001 35.897158) (width 0.2) (layer "B.Cu") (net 12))
 (segment (start 133.3 36.2) (end 137.7815 31.7185) (width 0.2) (layer "B.Cu") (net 12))
 (segment (start 133.3 39.9385) (end 133.3 36.2) (width 0.2) (layer "B.Cu") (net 12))
 (segment (start 137.7815 31.7185) (end 140.32 31.7185) (width 0.2) (layer "B.Cu") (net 12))
 (segment (start 109.6 79.35) (end 109.55 79.35) (width 0.2) (layer "F.Cu") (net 15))
 (segment (start 111.45 81.2) (end 109.6 79.35) (width 0.2) (layer "F.Cu") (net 15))
 (via (at 109.55 79.35) (size 0.6) (drill 0.3) (layers "F.Cu" "B.Cu") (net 15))
 (via (at 111.45 81.2) (size 0.6) (drill 0.3) (layers "F.Cu" "B.Cu") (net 15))
 (segment (start 107.45 79.35) (end 105.25 77.15) (width 0.2) (layer "B.Cu") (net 15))
 (segment (start 109.55 79.35) (end 107.45 79.35) (width 0.2) (layer "B.Cu") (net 15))
 (segment (start 111.497158 82.899999) (end 111.497158 81.247158) (width 0.2) (layer "B.Cu") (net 15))
 (segment (start 105.25 36.45) (end 107.302842 34.397158) (width 0.2) (layer "B.Cu") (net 15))
 (segment (start 111.497158 81.247158) (end 111.45 81.2) (width 0.2) (layer "B.Cu") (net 15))
 (segment (start 107.302842 34.397158) (end 109.350001 34.397158) (width 0.2) (layer "B.Cu") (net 15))
 (segment (start 105.25 77.15) (end 105.25 36.45) (width 0.2) (layer "B.Cu") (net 15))
 (segment (start 134.249999 82.95) (end 134.25 82.949999) (width 0.2) (layer "F.Cu") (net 14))
 (segment (start 126.95 82.95) (end 134.249999 82.95) (width 0.2) (layer "F.Cu") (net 14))
 (via (at 126.95 82.95) (size 0.6) (drill 0.3) (layers "F.Cu" "B.Cu") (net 14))
 (via (at 134.25 82.949999) (size 0.6) (drill 0.3) (layers "F.Cu" "B.Cu") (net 14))
 (segment (start 128.35 22.3) (end 130.1485 24.0985) (width 0.2) (layer "B.Cu") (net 14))
 (segment (start 110 80.65) (end 112 78.65) (width 0.2) (layer "B.Cu") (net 14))
 (segment (start 120.1 52.3) (end 120.1 46.2) (width 0.2) (layer "B.Cu") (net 14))
 (segment (start 112 78.65) (end 120.35 78.65) (width 0.2) (layer "B.Cu") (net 14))
 (segment (start 109.997158 82.899999) (end 110 82.897157) (width 0.2) (layer "B.Cu") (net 14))
 (segment (start 115.802842 34.397158) (end 116.15 34.05) (width 0.2) (layer "B.Cu") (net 14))
 (segment (start 121.45 53.65) (end 120.1 52.3) (width 0.2) (layer "B.Cu") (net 14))
 (segment (start 120.2 22.3) (end 128.35 22.3) (width 0.2) (layer "B.Cu") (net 14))
 (segment (start 150.9985 24.0985) (end 140.32 24.0985) (width 0.2) (layer "B.Cu") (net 14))
 (segment (start 121.45 77.45) (end 121.45 53.65) (width 0.2) (layer "B.Cu") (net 14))
 (segment (start 120.1 46.2) (end 116.15 42.25) (width 0.2) (layer "B.Cu") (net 14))
 (segment (start 116.15 26.35) (end 120.2 22.3) (width 0.2) (layer "B.Cu") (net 14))
 (segment (start 155.4875 34.4) (end 155.4875 28.5875) (width 0.2) (layer "B.Cu") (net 14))
 (segment (start 114.550001 34.397158) (end 115.802842 34.397158) (width 0.2) (layer "B.Cu") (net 14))
 (segment (start 120.35 78.65) (end 121.5 77.5) (width 0.2) (layer "B.Cu") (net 14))
 (segment (start 126.95 82.95) (end 121.5 77.5) (width 0.2) (layer "B.Cu") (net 14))
 (segment (start 130.1485 24.0985) (end 140.32 24.0985) (width 0.2) (layer "B.Cu") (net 14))
 (segment (start 116.15 34.05) (end 116.15 33.7) (width 0.2) (layer "B.Cu") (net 14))
 (segment (start 155.4875 28.5875) (end 150.9985 24.0985) (width 0.2) (layer "B.Cu") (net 14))
 (segment (start 110 82.897157) (end 110 80.65) (width 0.2) (layer "B.Cu") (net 14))
 (segment (start 134.25 82.949999) (end 149.997158 82.949999) (width 0.2) (layer "B.Cu") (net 14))
 (segment (start 116.15 33.7) (end 116.15 26.35) (width 0.2) (layer "B.Cu") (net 14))
 (segment (start 121.5 77.5) (end 121.45 77.45) (width 0.2) (layer "B.Cu") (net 14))
 (segment (start 116.15 42.25) (end 116.15 33.7) (width 0.2) (layer "B.Cu") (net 14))
 (segment (start 133.1 81.05) (end 124.55 89.6) (width 0.2) (layer "B.Cu") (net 18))
 (segment (start 109.997158 88.899999) (end 109.997158 88.099999) (width 0.2) (layer "B.Cu") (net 18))
 (segment (start 151.497158 82.149999) (end 150.397159 81.05) (width 0.2) (layer "B.Cu") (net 18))
 (segment (start 124.55 89.6) (end 110.697159 89.6) (width 0.2) (layer "B.Cu") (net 18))
 (segment (start 151.497158 82.949999) (end 151.497158 82.149999) (width 0.2) (layer "B.Cu") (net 18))
 (segment (start 110.697159 89.6) (end 109.997158 88.899999) (width 0.2) (layer "B.Cu") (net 18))
 (segment (start 150.397159 81.05) (end 133.1 81.05) (width 0.2) (layer "B.Cu") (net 18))
 (segment (start 160.7 84) (end 155.1 89.6) (width 0.2) (layer "B.Cu") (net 17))
 (segment (start 149.997158 88.149999) (end 149.997158 88.949999) (width 0.2) (layer "B.Cu") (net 17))
 (segment (start 159.3 35.9) (end 160.7 37.3) (width 0.2) (layer "B.Cu") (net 17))
 (segment (start 160.7 37.3) (end 160.7 84) (width 0.2) (layer "B.Cu") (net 17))
 (segment (start 155.4875 35.9) (end 159.3 35.9) (width 0.2) (layer "B.Cu") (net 17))
 (segment (start 150.647159 89.6) (end 155.1 89.6) (width 0.2) (layer "B.Cu") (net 17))
 (segment (start 149.997158 88.949999) (end 150.647159 89.6) (width 0.2) (layer "B.Cu") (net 17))
 (segment (start 106.45 30.05) (end 106.45 48.97) (width 0.2) (layer "F.Cu") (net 3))
 (segment (start 112.4015 24.0985) (end 106.45 30.05) (width 0.2) (layer "F.Cu") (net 3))
 (segment (start 106.45 48.97) (end 108.84 51.36) (width 0.2) (layer "F.Cu") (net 3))
 (segment (start 125.08 24.0985) (end 112.4015 24.0985) (width 0.2) (layer "F.Cu") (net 3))
 (segment (start 124.00237 26.6385) (end 125.08 26.6385) (width 0.2) (layer "F.Cu") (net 4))
 (segment (start 120.75 29.89087) (end 124.00237 26.6385) (width 0.2) (layer "F.Cu") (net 4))
 (segment (start 120.7 44.55) (end 120.7 55.85) (width 0.2) (layer "F.Cu") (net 4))
 (segment (start 119.7 43.55) (end 120.7 44.55) (width 0.2) (layer "F.Cu") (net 4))
 (segment (start 120.75 39.35) (end 120.75 29.89087) (width 0.2) (layer "F.Cu") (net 4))
 (via (at 120.7 55.85) (size 0.6) (drill 0.3) (layers "F.Cu" "B.Cu") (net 4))
 (via (at 120.75 39.35) (size 0.6) (drill 0.3) (layers "F.Cu" "B.Cu") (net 4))
 (via (at 119.7 43.55) (size 0.6) (drill 0.3) (layers "F.Cu" "B.Cu") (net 4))
 (segment (start 119.7 41.9) (end 119.7 43.55) (width 0.2) (layer "B.Cu") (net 4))
 (segment (start 112.05 69.2) (end 110.84 70.41) (width 0.2) (layer "B.Cu") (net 4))
 (segment (start 120.75 39.35) (end 120.75 40.85) (width 0.2) (layer "B.Cu") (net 4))
 (segment (start 112.05 69.2) (end 112.05 64.5) (width 0.2) (layer "B.Cu") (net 4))
 (segment (start 120.75 40.85) (end 119.7 41.9) (width 0.2) (layer "B.Cu") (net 4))
 (segment (start 112.05 64.5) (end 120.7 55.85) (width 0.2) (layer "B.Cu") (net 4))
 (segment (start 110.84 70.41) (end 108.86 70.41) (width 0.2) (layer "B.Cu") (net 4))
 (segment (start 125.08 29.1785) (end 127.0285 29.1785) (width 0.2) (layer "B.Cu") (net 5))
 (segment (start 131.15 33.3) (end 131.15 48.12) (width 0.2) (layer "B.Cu") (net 5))
 (segment (start 127.0285 29.1785) (end 131.15 33.3) (width 0.2) (layer "B.Cu") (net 5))
 (segment (start 131.15 48.12) (end 127.91 51.36) (width 0.2) (layer "B.Cu") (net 5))
 (segment (start 133.6685 31.7185) (end 136.15 34.2) (width 0.2) (layer "F.Cu") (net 6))
 (segment (start 137.2 35.25) (end 137.2 36.8) (width 0.2) (layer "F.Cu") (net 6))
 (segment (start 136.15 34.2) (end 137.2 35.25) (width 0.2) (layer "F.Cu") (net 6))
 (segment (start 125.08 31.7185) (end 133.6685 31.7185) (width 0.2) (layer "F.Cu") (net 6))
 (via (at 137.2 36.8) (size 0.6) (drill 0.3) (layers "F.Cu" "B.Cu") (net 6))
 (segment (start 129.44 70.41) (end 127.94 70.41) (width 0.2) (layer "B.Cu") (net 6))
 (segment (start 127.95 70.4) (end 127.94 70.41) (width 0.2) (layer "B.Cu") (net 6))
 (segment (start 134.75 51.2) (end 134.75 56.15) (width 0.2) (layer "B.Cu") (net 6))
 (segment (start 130.2 60.7) (end 130.2 69.65) (width 0.2) (layer "B.Cu") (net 6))
 (segment (start 137.2 48.75) (end 134.75 51.2) (width 0.2) (layer "B.Cu") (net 6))
 (segment (start 130.2 69.65) (end 129.44 70.41) (width 0.2) (layer "B.Cu") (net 6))
 (segment (start 137.2 36.8) (end 137.2 48.75) (width 0.2) (layer "B.Cu") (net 6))
 (segment (start 134.75 56.15) (end 130.2 60.7) (width 0.2) (layer "B.Cu") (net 6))
 (segment (start 146.95 47.95) (end 133.2585 34.2585) (width 0.2) (layer "F.Cu") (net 2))
 (segment (start 146.95 51.35) (end 146.95 47.95) (width 0.2) (layer "F.Cu") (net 2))
 (segment (start 133.2585 34.2585) (end 125.08 34.2585) (width 0.2) (layer "F.Cu") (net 2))
 (segment (start 138.23 41.33) (end 133.6985 36.7985) (width 0.2) (layer "F.Cu") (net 7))
 (segment (start 138.8 41.33) (end 138.23 41.33) (width 0.2) (layer "F.Cu") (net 7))
 (segment (start 133.6985 36.7985) (end 125.08 36.7985) (width 0.2) (layer "F.Cu") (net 7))
 (via (at 138.8 41.33) (size 0.6) (drill 0.3) (layers "F.Cu" "B.Cu") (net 7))
 (segment (start 142 69.2) (end 143.2 70.4) (width 0.2) (layer "B.Cu") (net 7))
 (segment (start 142 42.1) (end 142 69.2) (width 0.2) (layer "B.Cu") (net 7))
 (segment (start 138.8 41.33) (end 141.23 41.33) (width 0.2) (layer "B.Cu") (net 7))
 (segment (start 143.2 70.4) (end 146.95 70.4) (width 0.2) (layer "B.Cu") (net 7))
 (segment (start 141.23 41.33) (end 142 42.1) (width 0.2) (layer "B.Cu") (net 7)))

